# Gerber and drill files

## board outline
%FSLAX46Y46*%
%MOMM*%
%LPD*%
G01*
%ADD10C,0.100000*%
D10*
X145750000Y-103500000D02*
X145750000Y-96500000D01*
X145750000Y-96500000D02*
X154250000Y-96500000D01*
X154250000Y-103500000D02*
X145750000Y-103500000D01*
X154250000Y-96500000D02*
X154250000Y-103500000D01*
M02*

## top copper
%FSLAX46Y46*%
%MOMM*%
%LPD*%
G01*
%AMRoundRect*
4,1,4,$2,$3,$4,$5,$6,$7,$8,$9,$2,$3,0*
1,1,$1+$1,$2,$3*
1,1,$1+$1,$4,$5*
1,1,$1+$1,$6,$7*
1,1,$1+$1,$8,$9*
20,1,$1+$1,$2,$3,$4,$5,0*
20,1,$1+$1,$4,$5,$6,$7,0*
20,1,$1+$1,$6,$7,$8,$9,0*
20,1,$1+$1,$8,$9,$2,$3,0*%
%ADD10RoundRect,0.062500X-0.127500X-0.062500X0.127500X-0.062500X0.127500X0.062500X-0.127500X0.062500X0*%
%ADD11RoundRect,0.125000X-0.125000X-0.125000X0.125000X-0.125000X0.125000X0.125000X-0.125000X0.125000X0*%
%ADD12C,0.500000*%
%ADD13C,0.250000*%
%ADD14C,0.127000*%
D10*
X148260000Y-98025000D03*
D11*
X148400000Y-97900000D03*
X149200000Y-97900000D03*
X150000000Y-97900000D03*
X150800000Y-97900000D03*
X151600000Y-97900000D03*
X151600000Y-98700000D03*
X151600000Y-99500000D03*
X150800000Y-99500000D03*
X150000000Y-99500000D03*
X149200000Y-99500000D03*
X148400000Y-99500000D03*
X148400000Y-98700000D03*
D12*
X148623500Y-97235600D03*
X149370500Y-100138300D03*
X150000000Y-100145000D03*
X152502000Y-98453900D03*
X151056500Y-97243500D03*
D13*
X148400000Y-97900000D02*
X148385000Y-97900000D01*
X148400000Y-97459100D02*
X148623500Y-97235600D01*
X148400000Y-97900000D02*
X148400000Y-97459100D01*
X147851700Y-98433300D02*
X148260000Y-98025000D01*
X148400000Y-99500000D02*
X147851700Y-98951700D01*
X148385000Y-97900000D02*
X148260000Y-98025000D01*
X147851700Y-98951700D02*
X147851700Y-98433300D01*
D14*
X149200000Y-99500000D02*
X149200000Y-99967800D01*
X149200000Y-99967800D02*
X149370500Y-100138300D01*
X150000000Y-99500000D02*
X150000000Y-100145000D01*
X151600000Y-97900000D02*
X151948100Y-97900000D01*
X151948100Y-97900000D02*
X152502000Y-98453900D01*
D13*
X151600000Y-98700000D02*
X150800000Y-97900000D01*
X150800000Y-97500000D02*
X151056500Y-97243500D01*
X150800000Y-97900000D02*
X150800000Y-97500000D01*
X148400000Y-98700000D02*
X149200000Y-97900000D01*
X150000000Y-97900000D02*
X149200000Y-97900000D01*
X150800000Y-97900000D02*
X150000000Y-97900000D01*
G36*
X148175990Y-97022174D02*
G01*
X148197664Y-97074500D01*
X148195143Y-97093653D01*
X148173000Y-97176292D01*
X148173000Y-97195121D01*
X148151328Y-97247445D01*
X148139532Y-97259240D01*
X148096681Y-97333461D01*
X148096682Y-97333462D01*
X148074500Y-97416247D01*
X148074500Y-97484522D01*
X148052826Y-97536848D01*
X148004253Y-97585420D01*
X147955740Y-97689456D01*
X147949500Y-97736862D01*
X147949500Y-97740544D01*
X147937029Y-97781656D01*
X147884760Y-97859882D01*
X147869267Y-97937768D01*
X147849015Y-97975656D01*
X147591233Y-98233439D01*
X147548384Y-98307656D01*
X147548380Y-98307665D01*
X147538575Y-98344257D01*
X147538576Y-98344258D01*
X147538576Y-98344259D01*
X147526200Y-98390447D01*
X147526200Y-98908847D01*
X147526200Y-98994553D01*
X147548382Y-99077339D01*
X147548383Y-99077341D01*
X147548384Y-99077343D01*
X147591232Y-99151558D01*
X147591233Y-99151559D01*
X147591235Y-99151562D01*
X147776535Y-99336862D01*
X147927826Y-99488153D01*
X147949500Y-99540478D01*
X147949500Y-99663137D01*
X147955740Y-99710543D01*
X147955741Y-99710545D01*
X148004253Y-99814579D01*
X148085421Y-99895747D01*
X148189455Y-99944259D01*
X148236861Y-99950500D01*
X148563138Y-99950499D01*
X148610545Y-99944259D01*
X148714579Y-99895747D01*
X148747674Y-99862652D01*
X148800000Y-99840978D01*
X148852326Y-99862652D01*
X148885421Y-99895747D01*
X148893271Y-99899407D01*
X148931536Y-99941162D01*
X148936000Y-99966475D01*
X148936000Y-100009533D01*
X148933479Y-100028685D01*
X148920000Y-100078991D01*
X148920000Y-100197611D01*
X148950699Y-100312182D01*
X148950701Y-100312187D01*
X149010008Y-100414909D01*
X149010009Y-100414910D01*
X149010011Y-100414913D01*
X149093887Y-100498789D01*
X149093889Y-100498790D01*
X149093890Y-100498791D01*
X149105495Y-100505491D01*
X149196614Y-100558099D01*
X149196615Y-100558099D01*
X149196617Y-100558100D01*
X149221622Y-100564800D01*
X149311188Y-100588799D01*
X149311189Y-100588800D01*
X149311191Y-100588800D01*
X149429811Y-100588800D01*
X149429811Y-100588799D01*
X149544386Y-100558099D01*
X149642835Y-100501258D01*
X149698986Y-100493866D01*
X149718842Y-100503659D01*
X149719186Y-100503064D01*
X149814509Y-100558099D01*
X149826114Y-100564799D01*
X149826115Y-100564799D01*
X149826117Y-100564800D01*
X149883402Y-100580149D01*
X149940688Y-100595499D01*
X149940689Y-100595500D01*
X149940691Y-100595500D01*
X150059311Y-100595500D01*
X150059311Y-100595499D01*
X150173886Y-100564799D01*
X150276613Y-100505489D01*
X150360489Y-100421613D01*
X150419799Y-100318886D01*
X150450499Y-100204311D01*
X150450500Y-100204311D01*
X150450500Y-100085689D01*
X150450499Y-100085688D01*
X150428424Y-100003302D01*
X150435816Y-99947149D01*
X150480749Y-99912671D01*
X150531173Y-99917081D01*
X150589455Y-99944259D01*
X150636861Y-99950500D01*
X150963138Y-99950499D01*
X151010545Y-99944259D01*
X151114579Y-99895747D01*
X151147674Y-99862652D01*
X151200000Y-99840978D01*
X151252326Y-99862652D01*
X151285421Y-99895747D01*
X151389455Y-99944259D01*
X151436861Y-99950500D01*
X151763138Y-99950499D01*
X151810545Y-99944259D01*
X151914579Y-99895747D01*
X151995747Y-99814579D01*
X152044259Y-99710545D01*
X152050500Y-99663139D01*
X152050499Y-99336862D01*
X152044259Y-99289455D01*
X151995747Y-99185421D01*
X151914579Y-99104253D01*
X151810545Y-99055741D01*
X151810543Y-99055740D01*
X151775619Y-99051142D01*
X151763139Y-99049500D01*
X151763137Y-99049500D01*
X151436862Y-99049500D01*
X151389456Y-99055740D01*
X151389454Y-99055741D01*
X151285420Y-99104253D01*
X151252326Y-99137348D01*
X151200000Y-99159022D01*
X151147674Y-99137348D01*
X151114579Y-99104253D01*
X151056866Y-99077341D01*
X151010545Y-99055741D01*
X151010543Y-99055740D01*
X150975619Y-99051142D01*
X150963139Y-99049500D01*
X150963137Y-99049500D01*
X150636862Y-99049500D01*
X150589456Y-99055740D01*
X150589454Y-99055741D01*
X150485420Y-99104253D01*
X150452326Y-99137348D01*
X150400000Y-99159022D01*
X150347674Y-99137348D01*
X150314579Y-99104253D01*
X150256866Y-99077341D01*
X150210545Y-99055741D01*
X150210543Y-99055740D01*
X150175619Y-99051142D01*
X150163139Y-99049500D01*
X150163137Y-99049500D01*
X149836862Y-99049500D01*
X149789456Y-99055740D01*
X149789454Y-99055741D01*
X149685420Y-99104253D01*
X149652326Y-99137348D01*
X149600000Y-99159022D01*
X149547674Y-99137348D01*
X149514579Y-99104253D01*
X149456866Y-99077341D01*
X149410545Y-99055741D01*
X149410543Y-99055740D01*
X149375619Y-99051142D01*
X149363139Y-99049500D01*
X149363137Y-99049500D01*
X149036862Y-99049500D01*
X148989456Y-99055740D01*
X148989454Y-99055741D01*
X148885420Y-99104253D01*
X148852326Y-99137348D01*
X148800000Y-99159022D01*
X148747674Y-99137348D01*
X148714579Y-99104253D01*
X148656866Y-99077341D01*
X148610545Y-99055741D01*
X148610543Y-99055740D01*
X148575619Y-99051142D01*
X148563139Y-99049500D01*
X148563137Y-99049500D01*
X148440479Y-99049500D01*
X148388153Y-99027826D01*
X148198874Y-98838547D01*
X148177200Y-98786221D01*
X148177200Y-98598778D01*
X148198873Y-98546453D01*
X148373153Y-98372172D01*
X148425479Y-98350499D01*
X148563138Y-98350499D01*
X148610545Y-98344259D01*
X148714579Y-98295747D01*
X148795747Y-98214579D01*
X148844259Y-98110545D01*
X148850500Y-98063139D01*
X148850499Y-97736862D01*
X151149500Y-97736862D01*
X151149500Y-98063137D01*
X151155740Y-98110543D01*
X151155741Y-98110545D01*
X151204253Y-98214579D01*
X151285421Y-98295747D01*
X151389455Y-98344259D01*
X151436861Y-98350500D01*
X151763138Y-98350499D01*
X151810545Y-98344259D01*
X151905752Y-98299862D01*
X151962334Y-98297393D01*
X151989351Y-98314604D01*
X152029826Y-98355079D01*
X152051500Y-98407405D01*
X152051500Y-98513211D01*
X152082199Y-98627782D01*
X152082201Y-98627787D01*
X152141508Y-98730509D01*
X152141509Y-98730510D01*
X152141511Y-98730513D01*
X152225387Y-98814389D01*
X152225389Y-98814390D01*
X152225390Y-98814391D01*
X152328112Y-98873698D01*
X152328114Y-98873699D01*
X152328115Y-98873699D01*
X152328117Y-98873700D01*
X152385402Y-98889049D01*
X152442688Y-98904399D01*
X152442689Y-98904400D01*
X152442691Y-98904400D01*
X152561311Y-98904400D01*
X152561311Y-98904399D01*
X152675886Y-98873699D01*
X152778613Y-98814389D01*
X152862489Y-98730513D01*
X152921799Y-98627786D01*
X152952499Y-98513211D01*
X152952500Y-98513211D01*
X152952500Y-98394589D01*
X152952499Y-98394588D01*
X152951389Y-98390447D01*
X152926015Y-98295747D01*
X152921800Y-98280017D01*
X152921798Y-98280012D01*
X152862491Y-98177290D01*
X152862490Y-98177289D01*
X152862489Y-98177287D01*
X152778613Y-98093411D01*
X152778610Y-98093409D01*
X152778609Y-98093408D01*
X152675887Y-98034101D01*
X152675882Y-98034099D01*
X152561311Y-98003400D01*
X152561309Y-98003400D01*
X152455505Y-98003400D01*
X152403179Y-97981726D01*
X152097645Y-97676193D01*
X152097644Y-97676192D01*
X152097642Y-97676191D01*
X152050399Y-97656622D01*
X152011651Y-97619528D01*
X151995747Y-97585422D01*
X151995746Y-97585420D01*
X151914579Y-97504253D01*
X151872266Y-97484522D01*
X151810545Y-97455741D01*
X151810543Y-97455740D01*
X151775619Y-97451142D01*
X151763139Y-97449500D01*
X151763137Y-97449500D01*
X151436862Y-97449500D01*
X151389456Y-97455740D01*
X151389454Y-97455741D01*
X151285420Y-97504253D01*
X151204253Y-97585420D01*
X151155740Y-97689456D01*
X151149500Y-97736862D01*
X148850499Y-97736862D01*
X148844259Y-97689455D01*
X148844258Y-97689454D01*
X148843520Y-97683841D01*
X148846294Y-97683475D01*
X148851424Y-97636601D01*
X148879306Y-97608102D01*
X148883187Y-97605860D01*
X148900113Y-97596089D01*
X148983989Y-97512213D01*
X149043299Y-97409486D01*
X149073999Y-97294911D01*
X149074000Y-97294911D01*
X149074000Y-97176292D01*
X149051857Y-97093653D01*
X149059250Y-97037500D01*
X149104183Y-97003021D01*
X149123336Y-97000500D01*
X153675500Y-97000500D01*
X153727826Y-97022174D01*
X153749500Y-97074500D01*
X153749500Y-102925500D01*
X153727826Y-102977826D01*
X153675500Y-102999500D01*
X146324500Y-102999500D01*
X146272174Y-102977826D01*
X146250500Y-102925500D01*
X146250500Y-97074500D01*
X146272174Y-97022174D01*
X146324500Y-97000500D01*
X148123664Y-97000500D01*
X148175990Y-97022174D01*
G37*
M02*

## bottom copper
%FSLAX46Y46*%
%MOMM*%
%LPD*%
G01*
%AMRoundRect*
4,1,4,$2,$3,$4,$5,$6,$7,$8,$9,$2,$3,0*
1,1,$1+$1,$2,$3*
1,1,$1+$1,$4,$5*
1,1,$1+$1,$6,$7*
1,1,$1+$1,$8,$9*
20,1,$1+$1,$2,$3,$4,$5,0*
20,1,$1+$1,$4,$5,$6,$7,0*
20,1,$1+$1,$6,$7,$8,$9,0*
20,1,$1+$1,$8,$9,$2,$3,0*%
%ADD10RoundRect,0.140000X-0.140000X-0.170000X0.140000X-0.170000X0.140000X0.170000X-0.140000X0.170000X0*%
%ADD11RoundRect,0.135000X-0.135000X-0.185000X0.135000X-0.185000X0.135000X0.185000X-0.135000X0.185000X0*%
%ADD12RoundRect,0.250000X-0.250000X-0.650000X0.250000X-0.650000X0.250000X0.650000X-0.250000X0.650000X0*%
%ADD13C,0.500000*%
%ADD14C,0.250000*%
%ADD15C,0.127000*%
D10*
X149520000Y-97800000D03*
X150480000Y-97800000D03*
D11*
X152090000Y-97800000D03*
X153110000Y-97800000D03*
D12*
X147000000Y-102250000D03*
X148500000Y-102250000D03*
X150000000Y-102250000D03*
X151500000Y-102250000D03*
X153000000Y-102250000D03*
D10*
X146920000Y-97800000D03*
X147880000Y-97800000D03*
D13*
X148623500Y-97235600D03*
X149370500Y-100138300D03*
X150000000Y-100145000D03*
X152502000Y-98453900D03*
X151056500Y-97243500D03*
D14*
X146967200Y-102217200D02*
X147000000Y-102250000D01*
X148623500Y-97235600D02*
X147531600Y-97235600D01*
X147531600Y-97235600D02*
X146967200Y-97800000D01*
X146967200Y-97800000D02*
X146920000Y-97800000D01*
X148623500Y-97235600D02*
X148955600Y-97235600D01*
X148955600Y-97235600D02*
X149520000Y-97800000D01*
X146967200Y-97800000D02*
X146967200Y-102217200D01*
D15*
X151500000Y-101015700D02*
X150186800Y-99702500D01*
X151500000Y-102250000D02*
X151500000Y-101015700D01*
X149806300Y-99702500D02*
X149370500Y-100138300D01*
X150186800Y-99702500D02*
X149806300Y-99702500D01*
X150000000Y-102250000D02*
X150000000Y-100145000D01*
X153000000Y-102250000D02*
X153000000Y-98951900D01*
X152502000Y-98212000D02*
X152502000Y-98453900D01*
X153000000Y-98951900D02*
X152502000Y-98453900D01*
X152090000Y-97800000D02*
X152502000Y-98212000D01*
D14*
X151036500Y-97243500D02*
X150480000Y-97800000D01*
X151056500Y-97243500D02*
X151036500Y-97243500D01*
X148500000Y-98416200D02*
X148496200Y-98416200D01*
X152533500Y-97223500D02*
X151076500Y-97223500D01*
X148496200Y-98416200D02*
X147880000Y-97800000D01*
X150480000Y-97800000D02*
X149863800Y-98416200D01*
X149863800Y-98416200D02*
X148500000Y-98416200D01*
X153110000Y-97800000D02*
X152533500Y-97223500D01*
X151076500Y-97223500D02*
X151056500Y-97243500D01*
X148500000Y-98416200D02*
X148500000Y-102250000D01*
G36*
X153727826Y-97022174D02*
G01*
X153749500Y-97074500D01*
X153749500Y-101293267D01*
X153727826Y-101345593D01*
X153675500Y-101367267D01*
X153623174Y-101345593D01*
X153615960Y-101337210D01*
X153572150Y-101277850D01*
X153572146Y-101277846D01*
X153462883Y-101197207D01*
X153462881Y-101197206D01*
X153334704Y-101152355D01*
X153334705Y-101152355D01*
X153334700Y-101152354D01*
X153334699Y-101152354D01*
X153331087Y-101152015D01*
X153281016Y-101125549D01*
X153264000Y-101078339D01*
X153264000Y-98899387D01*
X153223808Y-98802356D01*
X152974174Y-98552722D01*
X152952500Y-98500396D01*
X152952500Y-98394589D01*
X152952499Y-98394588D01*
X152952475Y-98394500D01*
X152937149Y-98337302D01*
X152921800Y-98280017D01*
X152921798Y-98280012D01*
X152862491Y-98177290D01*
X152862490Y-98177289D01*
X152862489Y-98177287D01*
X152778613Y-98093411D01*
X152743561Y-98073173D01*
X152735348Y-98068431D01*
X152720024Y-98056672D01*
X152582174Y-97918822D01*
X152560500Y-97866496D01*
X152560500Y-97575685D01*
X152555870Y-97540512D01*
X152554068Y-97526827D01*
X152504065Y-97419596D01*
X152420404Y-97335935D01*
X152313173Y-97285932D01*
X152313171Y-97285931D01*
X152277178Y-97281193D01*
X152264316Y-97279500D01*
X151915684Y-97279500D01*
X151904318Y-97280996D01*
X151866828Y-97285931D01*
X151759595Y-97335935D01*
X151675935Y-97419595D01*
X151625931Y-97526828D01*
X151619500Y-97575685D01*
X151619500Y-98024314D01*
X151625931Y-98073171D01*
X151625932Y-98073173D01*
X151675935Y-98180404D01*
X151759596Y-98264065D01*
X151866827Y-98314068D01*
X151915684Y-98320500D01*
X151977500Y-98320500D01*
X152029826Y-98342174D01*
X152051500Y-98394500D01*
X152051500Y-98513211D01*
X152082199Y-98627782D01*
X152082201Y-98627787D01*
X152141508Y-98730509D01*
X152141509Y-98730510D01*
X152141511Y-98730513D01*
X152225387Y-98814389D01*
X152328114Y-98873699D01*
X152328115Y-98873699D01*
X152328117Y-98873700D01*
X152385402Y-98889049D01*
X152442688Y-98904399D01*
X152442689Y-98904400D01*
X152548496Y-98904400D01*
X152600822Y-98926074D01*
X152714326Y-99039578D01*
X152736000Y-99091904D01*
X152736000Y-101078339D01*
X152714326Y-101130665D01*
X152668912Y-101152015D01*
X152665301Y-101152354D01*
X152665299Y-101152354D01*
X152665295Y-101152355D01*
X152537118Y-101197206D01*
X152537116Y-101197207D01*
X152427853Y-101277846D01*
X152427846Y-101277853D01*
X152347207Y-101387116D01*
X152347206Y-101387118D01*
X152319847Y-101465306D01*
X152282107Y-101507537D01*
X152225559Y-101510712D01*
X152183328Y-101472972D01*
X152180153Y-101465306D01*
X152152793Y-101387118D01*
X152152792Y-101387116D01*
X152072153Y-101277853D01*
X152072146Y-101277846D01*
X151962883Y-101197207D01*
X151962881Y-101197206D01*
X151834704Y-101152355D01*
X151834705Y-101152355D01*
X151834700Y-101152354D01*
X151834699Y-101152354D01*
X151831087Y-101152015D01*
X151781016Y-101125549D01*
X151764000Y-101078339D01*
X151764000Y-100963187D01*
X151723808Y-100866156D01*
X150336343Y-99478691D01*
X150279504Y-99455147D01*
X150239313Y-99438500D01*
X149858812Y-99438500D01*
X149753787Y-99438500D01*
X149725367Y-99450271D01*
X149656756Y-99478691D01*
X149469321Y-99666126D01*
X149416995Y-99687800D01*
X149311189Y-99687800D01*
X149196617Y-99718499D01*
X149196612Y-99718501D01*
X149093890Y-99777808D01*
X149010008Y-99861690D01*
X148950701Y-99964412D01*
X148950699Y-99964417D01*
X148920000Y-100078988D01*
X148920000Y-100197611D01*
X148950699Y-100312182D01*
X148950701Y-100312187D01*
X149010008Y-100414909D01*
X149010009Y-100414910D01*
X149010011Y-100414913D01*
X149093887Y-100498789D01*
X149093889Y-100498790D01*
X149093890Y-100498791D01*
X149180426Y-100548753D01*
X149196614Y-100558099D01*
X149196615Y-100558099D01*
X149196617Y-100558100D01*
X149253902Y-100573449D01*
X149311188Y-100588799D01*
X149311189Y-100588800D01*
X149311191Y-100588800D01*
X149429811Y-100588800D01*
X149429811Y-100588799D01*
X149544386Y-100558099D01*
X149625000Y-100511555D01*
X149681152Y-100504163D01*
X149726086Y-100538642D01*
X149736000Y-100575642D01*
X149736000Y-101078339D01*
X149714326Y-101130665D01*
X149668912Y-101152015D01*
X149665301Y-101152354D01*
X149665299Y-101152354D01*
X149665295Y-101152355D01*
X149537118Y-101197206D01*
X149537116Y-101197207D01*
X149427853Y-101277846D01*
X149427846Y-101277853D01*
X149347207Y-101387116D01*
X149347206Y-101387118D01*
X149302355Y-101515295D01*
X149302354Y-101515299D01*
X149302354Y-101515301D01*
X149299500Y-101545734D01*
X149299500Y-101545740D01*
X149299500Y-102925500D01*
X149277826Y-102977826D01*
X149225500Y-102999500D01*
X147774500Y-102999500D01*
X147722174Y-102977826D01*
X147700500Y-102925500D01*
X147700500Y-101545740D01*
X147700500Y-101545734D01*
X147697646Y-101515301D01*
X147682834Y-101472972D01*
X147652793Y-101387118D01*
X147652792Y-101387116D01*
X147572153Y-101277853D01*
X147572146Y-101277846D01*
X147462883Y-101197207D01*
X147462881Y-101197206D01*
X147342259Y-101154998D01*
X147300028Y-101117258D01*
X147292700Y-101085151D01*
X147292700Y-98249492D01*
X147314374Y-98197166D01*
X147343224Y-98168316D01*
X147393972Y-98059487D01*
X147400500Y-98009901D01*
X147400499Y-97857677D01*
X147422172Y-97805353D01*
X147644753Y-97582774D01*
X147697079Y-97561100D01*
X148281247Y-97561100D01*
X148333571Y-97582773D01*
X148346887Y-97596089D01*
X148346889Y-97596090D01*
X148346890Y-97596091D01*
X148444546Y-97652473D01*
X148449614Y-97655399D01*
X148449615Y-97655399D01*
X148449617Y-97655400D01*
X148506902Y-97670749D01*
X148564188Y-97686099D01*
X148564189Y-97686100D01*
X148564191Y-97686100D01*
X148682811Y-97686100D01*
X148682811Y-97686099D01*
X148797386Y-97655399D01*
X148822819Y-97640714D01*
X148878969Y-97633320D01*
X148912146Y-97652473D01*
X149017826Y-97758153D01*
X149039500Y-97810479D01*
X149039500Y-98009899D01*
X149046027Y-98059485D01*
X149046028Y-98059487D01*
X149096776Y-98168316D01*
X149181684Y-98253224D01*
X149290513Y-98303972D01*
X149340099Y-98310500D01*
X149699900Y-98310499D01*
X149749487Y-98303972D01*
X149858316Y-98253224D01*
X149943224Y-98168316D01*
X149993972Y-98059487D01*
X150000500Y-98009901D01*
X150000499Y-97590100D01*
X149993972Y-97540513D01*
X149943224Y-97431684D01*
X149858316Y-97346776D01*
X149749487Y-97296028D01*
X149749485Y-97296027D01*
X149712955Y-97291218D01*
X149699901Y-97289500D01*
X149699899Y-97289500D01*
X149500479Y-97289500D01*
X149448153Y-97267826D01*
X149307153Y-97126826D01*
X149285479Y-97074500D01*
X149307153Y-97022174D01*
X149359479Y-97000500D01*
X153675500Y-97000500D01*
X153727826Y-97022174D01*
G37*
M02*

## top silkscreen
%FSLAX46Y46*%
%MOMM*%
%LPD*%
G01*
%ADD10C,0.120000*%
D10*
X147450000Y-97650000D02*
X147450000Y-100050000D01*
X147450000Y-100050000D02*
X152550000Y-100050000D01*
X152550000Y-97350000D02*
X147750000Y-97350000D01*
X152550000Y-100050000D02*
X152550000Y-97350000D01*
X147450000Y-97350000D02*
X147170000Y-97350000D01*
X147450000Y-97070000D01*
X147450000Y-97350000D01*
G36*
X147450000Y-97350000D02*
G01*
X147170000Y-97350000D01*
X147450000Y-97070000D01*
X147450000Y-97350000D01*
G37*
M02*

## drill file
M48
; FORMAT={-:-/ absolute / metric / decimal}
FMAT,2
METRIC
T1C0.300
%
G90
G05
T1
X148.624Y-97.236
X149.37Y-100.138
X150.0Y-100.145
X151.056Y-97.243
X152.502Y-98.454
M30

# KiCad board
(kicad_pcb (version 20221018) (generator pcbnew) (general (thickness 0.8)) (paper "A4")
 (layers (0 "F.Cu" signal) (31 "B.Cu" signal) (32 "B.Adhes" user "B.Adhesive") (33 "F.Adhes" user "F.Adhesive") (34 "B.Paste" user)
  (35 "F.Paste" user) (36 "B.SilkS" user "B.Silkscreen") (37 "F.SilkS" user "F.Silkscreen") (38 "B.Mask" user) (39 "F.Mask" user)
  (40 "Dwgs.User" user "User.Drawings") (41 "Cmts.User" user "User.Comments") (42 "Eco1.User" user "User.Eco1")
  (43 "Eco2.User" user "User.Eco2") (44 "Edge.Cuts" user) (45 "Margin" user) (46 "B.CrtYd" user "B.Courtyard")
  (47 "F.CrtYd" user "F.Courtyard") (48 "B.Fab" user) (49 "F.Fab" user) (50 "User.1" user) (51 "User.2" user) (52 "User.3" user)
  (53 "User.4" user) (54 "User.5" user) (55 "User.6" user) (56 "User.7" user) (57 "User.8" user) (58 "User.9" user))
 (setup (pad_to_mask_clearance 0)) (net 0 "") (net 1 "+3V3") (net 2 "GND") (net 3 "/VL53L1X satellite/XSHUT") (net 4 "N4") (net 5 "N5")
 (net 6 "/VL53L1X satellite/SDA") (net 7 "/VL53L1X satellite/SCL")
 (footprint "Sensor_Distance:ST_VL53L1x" (layer "F.Cu") (at 150 98.7)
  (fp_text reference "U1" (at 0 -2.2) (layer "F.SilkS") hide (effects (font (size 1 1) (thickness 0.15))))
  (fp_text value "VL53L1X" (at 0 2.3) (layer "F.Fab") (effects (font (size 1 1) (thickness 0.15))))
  (fp_line (start -2.55 -1.05) (end -2.55 1.35) (stroke (width 0.12) (type solid)) (layer "F.SilkS"))
  (fp_line (start -2.55 1.35) (end 2.55 1.35) (stroke (width 0.12) (type solid)) (layer "F.SilkS"))
  (fp_line (start 2.55 -1.35) (end -2.25 -1.35) (stroke (width 0.12) (type solid)) (layer "F.SilkS"))
  (fp_line (start 2.55 1.35) (end 2.55 -1.35) (stroke (width 0.12) (type solid)) (layer "F.SilkS"))
  (fp_poly
   (pts (xy -2.55 -1.35) (xy -2.83 -1.35) (xy -2.55 -1.63) (xy -2.55 -1.35)) (stroke (width 0.12) (type solid)) (fill solid)
   (layer "F.SilkS"))
  (pad "1" smd roundrect (at -1.74 -0.675) (size 0.38 0.25) (layers "F.Cu" "F.Paste" "F.Mask") (roundrect_rratio 0.25) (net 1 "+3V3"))
  (pad "1" smd roundrect (at -1.6 -0.8) (size 0.5 0.5) (layers "F.Cu" "F.Paste" "F.Mask") (roundrect_rratio 0.25) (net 1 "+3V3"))
  (pad "2" smd roundrect (at -0.8 -0.8) (size 0.5 0.5) (layers "F.Cu" "F.Paste" "F.Mask") (roundrect_rratio 0.25) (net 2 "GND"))
  (pad "3" smd roundrect (at 0 -0.8) (size 0.5 0.5) (layers "F.Cu" "F.Paste" "F.Mask") (roundrect_rratio 0.25) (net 2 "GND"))
  (pad "4" smd roundrect (at 0.8 -0.8) (size 0.5 0.5) (layers "F.Cu" "F.Paste" "F.Mask") (roundrect_rratio 0.25) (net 2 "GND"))
  (pad "5" smd roundrect (at 1.6 -0.8) (size 0.5 0.5) (layers "F.Cu" "F.Paste" "F.Mask") (roundrect_rratio 0.25)
   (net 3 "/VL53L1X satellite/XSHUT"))
  (pad "6" smd roundrect (at 1.6 0) (size 0.5 0.5) (layers "F.Cu" "F.Paste" "F.Mask") (roundrect_rratio 0.25) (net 2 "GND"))
  (pad "7" smd roundrect (at 1.6 0.8) (size 0.5 0.5) (layers "F.Cu" "F.Paste" "F.Mask") (roundrect_rratio 0.25) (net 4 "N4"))
  (pad "8" smd roundrect (at 0.8 0.8) (size 0.5 0.5) (layers "F.Cu" "F.Paste" "F.Mask") (roundrect_rratio 0.25) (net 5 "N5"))
  (pad "9" smd roundrect (at 0 0.8) (size 0.5 0.5) (layers "F.Cu" "F.Paste" "F.Mask") (roundrect_rratio 0.25)
   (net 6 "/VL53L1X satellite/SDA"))
  (pad "10" smd roundrect (at -0.8 0.8) (size 0.5 0.5) (layers "F.Cu" "F.Paste" "F.Mask") (roundrect_rratio 0.25)
   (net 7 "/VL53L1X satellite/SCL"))
  (pad "11" smd roundrect (at -1.6 0.8) (size 0.5 0.5) (layers "F.Cu" "F.Paste" "F.Mask") (roundrect_rratio 0.25) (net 1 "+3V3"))
  (pad "12" smd roundrect (at -1.6 0) (size 0.5 0.5) (layers "F.Cu" "F.Paste" "F.Mask") (roundrect_rratio 0.25) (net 2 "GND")))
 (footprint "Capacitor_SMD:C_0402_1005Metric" (layer "B.Cu") (at 150 97.8)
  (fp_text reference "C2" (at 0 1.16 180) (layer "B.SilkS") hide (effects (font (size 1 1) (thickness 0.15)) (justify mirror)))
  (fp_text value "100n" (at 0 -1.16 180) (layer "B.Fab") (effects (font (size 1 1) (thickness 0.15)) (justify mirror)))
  (pad "1" smd roundrect (at -0.48 0) (size 0.56 0.62) (layers "B.Cu" "B.Paste" "B.Mask") (roundrect_rratio 0.25) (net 1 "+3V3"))
  (pad "2" smd roundrect (at 0.48 0) (size 0.56 0.62) (layers "B.Cu" "B.Paste" "B.Mask") (roundrect_rratio 0.25) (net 2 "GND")))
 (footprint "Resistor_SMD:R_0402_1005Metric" (layer "B.Cu") (at 152.6 97.8)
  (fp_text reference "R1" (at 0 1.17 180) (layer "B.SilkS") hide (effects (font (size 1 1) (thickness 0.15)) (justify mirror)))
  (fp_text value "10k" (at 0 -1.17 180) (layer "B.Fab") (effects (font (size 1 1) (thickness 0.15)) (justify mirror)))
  (pad "1" smd roundrect (at -0.51 0) (size 0.54 0.64) (layers "B.Cu" "B.Paste" "B.Mask") (roundrect_rratio 0.25)
   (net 3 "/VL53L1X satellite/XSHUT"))
  (pad "2" smd roundrect (at 0.51 0) (size 0.54 0.64) (layers "B.Cu" "B.Paste" "B.Mask") (roundrect_rratio 0.25) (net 2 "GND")))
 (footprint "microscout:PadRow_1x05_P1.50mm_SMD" (layer "B.Cu") (at 150 102.25)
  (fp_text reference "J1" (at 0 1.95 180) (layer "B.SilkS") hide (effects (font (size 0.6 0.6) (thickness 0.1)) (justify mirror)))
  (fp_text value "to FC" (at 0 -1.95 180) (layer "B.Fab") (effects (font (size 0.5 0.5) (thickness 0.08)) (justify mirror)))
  (pad "1" smd roundrect (at -3 0) (size 1 1.8) (layers "B.Cu" "B.Paste" "B.Mask") (roundrect_rratio 0.25) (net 1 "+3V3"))
  (pad "2" smd roundrect (at -1.5 0) (size 1 1.8) (layers "B.Cu" "B.Paste" "B.Mask") (roundrect_rratio 0.25) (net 2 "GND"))
  (pad "3" smd roundrect (at 0 0) (size 1 1.8) (layers "B.Cu" "B.Paste" "B.Mask") (roundrect_rratio 0.25) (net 6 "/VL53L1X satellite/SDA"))
  (pad "4" smd roundrect (at 1.5 0) (size 1 1.8) (layers "B.Cu" "B.Paste" "B.Mask") (roundrect_rratio 0.25) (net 7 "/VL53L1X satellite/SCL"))
  (pad "5" smd roundrect (at 3 0) (size 1 1.8) (layers "B.Cu" "B.Paste" "B.Mask") (roundrect_rratio 0.25) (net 3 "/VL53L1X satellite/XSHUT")))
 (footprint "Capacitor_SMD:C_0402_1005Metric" (layer "B.Cu") (at 147.4 97.8)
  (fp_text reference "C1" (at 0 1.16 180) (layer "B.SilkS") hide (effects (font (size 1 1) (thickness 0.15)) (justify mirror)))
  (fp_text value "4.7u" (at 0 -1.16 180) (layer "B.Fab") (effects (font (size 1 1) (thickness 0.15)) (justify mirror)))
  (pad "1" smd roundrect (at -0.48 0) (size 0.56 0.62) (layers "B.Cu" "B.Paste" "B.Mask") (roundrect_rratio 0.25) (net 1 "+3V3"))
  (pad "2" smd roundrect (at 0.48 0) (size 0.56 0.62) (layers "B.Cu" "B.Paste" "B.Mask") (roundrect_rratio 0.25) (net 2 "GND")))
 (gr_line (start 145.75 103.5) (end 145.75 96.5) (stroke (width 0.1) (type default)) (layer "Edge.Cuts"))
 (gr_line (start 145.75 96.5) (end 154.25 96.5) (stroke (width 0.1) (type default)) (layer "Edge.Cuts"))
 (gr_line (start 154.25 103.5) (end 145.75 103.5) (stroke (width 0.1) (type default)) (layer "Edge.Cuts"))
 (gr_line (start 154.25 96.5) (end 154.25 103.5) (stroke (width 0.1) (type default)) (layer "Edge.Cuts"))
 (segment (start 148.4 97.9) (end 148.385 97.9) (width 0.25) (layer "F.Cu") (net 1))
 (segment (start 148.4 97.4591) (end 148.6235 97.2356) (width 0.25) (layer "F.Cu") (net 1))
 (segment (start 148.4 97.9) (end 148.4 97.4591) (width 0.25) (layer "F.Cu") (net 1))
 (segment (start 147.8517 98.4333) (end 148.26 98.025) (width 0.25) (layer "F.Cu") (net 1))
 (segment (start 148.4 99.5) (end 147.8517 98.9517) (width 0.25) (layer "F.Cu") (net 1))
 (segment (start 148.385 97.9) (end 148.26 98.025) (width 0.25) (layer "F.Cu") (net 1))
 (segment (start 147.8517 98.9517) (end 147.8517 98.4333) (width 0.25) (layer "F.Cu") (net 1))
 (via (at 148.6235 97.2356) (size 0.5) (drill 0.3) (layers "F.Cu" "B.Cu") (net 1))
 (segment (start 146.9672 102.2172) (end 147 102.25) (width 0.25) (layer "B.Cu") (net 1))
 (segment (start 148.6235 97.2356) (end 147.5316 97.2356) (width 0.25) (layer "B.Cu") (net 1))
 (segment (start 147.5316 97.2356) (end 146.9672 97.8) (width 0.25) (layer "B.Cu") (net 1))
 (segment (start 146.9672 97.8) (end 146.92 97.8) (width 0.25) (layer "B.Cu") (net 1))
 (segment (start 148.6235 97.2356) (end 148.9556 97.2356) (width 0.25) (layer "B.Cu") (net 1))
 (segment (start 148.9556 97.2356) (end 149.52 97.8) (width 0.25) (layer "B.Cu") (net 1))
 (segment (start 146.9672 97.8) (end 146.9672 102.2172) (width 0.25) (layer "B.Cu") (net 1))
 (segment (start 149.2 99.5) (end 149.2 99.9678) (width 0.127) (layer "F.Cu") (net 7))
 (segment (start 149.2 99.9678) (end 149.3705 100.1383) (width 0.127) (layer "F.Cu") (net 7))
 (via (at 149.3705 100.1383) (size 0.5) (drill 0.3) (layers "F.Cu" "B.Cu") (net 7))
 (segment (start 151.5 101.0157) (end 150.1868 99.7025) (width 0.127) (layer "B.Cu") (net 7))
 (segment (start 151.5 102.25) (end 151.5 101.0157) (width 0.127) (layer "B.Cu") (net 7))
 (segment (start 149.8063 99.7025) (end 149.3705 100.1383) (width 0.127) (layer "B.Cu") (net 7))
 (segment (start 150.1868 99.7025) (end 149.8063 99.7025) (width 0.127) (layer "B.Cu") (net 7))
 (segment (start 150 99.5) (end 150 100.145) (width 0.127) (layer "F.Cu") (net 6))
 (via (at 150 100.145) (size 0.5) (drill 0.3) (layers "F.Cu" "B.Cu") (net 6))
 (segment (start 150 102.25) (end 150 100.145) (width 0.127) (layer "B.Cu") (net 6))
 (segment (start 151.6 97.9) (end 151.9481 97.9) (width 0.127) (layer "F.Cu") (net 3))
 (segment (start 151.9481 97.9) (end 152.502 98.4539) (width 0.127) (layer "F.Cu") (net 3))
 (via (at 152.502 98.4539) (size 0.5) (drill 0.3) (layers "F.Cu" "B.Cu") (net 3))
 (segment (start 153 102.25) (end 153 98.9519) (width 0.127) (layer "B.Cu") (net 3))
 (segment (start 152.502 98.212) (end 152.502 98.4539) (width 0.127) (layer "B.Cu") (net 3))
 (segment (start 153 98.9519) (end 152.502 98.4539) (width 0.127) (layer "B.Cu") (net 3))
 (segment (start 152.09 97.8) (end 152.502 98.212) (width 0.127) (layer "B.Cu") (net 3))
 (segment (start 151.6 98.7) (end 150.8 97.9) (width 0.25) (layer "F.Cu") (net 2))
 (segment (start 150.8 97.5) (end 151.0565 97.2435) (width 0.25) (layer "F.Cu") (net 2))
 (segment (start 150.8 97.9) (end 150.8 97.5) (width 0.25) (layer "F.Cu") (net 2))
 (segment (start 148.4 98.7) (end 149.2 97.9) (width 0.25) (layer "F.Cu") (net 2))
 (segment (start 150 97.9) (end 149.2 97.9) (width 0.25) (layer "F.Cu") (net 2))
 (segment (start 150.8 97.9) (end 150 97.9) (width 0.25) (layer "F.Cu") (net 2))
 (via (at 151.0565 97.2435) (size 0.5) (drill 0.3) (layers "F.Cu" "B.Cu") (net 2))
 (segment (start 151.0365 97.2435) (end 150.48 97.8) (width 0.25) (layer "B.Cu") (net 2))
 (segment (start 151.0565 97.2435) (end 151.0365 97.2435) (width 0.25) (layer "B.Cu") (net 2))
 (segment (start 148.5 98.4162) (end 148.4962 98.4162) (width 0.25) (layer "B.Cu") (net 2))
 (segment (start 152.5335 97.2235) (end 151.0765 97.2235) (width 0.25) (layer "B.Cu") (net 2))
 (segment (start 148.4962 98.4162) (end 147.88 97.8) (width 0.25) (layer "B.Cu") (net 2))
 (segment (start 150.48 97.8) (end 149.8638 98.4162) (width 0.25) (layer "B.Cu") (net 2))
 (segment (start 149.8638 98.4162) (end 148.5 98.4162) (width 0.25) (layer "B.Cu") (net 2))
 (segment (start 153.11 97.8) (end 152.5335 97.2235) (width 0.25) (layer "B.Cu") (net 2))
 (segment (start 151.0765 97.2235) (end 151.0565 97.2435) (width 0.25) (layer "B.Cu") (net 2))
 (segment (start 148.5 98.4162) (end 148.5 102.25) (width 0.25) (layer "B.Cu") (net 2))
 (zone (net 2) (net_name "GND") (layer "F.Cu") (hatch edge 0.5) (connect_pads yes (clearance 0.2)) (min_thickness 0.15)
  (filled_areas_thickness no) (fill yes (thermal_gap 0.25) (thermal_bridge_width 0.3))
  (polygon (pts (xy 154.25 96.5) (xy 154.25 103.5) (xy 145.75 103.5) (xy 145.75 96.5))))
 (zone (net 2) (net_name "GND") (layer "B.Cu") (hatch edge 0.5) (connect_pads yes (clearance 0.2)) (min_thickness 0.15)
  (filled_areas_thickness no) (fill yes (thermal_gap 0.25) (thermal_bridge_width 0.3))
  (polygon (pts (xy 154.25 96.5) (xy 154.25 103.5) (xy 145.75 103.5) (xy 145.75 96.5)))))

